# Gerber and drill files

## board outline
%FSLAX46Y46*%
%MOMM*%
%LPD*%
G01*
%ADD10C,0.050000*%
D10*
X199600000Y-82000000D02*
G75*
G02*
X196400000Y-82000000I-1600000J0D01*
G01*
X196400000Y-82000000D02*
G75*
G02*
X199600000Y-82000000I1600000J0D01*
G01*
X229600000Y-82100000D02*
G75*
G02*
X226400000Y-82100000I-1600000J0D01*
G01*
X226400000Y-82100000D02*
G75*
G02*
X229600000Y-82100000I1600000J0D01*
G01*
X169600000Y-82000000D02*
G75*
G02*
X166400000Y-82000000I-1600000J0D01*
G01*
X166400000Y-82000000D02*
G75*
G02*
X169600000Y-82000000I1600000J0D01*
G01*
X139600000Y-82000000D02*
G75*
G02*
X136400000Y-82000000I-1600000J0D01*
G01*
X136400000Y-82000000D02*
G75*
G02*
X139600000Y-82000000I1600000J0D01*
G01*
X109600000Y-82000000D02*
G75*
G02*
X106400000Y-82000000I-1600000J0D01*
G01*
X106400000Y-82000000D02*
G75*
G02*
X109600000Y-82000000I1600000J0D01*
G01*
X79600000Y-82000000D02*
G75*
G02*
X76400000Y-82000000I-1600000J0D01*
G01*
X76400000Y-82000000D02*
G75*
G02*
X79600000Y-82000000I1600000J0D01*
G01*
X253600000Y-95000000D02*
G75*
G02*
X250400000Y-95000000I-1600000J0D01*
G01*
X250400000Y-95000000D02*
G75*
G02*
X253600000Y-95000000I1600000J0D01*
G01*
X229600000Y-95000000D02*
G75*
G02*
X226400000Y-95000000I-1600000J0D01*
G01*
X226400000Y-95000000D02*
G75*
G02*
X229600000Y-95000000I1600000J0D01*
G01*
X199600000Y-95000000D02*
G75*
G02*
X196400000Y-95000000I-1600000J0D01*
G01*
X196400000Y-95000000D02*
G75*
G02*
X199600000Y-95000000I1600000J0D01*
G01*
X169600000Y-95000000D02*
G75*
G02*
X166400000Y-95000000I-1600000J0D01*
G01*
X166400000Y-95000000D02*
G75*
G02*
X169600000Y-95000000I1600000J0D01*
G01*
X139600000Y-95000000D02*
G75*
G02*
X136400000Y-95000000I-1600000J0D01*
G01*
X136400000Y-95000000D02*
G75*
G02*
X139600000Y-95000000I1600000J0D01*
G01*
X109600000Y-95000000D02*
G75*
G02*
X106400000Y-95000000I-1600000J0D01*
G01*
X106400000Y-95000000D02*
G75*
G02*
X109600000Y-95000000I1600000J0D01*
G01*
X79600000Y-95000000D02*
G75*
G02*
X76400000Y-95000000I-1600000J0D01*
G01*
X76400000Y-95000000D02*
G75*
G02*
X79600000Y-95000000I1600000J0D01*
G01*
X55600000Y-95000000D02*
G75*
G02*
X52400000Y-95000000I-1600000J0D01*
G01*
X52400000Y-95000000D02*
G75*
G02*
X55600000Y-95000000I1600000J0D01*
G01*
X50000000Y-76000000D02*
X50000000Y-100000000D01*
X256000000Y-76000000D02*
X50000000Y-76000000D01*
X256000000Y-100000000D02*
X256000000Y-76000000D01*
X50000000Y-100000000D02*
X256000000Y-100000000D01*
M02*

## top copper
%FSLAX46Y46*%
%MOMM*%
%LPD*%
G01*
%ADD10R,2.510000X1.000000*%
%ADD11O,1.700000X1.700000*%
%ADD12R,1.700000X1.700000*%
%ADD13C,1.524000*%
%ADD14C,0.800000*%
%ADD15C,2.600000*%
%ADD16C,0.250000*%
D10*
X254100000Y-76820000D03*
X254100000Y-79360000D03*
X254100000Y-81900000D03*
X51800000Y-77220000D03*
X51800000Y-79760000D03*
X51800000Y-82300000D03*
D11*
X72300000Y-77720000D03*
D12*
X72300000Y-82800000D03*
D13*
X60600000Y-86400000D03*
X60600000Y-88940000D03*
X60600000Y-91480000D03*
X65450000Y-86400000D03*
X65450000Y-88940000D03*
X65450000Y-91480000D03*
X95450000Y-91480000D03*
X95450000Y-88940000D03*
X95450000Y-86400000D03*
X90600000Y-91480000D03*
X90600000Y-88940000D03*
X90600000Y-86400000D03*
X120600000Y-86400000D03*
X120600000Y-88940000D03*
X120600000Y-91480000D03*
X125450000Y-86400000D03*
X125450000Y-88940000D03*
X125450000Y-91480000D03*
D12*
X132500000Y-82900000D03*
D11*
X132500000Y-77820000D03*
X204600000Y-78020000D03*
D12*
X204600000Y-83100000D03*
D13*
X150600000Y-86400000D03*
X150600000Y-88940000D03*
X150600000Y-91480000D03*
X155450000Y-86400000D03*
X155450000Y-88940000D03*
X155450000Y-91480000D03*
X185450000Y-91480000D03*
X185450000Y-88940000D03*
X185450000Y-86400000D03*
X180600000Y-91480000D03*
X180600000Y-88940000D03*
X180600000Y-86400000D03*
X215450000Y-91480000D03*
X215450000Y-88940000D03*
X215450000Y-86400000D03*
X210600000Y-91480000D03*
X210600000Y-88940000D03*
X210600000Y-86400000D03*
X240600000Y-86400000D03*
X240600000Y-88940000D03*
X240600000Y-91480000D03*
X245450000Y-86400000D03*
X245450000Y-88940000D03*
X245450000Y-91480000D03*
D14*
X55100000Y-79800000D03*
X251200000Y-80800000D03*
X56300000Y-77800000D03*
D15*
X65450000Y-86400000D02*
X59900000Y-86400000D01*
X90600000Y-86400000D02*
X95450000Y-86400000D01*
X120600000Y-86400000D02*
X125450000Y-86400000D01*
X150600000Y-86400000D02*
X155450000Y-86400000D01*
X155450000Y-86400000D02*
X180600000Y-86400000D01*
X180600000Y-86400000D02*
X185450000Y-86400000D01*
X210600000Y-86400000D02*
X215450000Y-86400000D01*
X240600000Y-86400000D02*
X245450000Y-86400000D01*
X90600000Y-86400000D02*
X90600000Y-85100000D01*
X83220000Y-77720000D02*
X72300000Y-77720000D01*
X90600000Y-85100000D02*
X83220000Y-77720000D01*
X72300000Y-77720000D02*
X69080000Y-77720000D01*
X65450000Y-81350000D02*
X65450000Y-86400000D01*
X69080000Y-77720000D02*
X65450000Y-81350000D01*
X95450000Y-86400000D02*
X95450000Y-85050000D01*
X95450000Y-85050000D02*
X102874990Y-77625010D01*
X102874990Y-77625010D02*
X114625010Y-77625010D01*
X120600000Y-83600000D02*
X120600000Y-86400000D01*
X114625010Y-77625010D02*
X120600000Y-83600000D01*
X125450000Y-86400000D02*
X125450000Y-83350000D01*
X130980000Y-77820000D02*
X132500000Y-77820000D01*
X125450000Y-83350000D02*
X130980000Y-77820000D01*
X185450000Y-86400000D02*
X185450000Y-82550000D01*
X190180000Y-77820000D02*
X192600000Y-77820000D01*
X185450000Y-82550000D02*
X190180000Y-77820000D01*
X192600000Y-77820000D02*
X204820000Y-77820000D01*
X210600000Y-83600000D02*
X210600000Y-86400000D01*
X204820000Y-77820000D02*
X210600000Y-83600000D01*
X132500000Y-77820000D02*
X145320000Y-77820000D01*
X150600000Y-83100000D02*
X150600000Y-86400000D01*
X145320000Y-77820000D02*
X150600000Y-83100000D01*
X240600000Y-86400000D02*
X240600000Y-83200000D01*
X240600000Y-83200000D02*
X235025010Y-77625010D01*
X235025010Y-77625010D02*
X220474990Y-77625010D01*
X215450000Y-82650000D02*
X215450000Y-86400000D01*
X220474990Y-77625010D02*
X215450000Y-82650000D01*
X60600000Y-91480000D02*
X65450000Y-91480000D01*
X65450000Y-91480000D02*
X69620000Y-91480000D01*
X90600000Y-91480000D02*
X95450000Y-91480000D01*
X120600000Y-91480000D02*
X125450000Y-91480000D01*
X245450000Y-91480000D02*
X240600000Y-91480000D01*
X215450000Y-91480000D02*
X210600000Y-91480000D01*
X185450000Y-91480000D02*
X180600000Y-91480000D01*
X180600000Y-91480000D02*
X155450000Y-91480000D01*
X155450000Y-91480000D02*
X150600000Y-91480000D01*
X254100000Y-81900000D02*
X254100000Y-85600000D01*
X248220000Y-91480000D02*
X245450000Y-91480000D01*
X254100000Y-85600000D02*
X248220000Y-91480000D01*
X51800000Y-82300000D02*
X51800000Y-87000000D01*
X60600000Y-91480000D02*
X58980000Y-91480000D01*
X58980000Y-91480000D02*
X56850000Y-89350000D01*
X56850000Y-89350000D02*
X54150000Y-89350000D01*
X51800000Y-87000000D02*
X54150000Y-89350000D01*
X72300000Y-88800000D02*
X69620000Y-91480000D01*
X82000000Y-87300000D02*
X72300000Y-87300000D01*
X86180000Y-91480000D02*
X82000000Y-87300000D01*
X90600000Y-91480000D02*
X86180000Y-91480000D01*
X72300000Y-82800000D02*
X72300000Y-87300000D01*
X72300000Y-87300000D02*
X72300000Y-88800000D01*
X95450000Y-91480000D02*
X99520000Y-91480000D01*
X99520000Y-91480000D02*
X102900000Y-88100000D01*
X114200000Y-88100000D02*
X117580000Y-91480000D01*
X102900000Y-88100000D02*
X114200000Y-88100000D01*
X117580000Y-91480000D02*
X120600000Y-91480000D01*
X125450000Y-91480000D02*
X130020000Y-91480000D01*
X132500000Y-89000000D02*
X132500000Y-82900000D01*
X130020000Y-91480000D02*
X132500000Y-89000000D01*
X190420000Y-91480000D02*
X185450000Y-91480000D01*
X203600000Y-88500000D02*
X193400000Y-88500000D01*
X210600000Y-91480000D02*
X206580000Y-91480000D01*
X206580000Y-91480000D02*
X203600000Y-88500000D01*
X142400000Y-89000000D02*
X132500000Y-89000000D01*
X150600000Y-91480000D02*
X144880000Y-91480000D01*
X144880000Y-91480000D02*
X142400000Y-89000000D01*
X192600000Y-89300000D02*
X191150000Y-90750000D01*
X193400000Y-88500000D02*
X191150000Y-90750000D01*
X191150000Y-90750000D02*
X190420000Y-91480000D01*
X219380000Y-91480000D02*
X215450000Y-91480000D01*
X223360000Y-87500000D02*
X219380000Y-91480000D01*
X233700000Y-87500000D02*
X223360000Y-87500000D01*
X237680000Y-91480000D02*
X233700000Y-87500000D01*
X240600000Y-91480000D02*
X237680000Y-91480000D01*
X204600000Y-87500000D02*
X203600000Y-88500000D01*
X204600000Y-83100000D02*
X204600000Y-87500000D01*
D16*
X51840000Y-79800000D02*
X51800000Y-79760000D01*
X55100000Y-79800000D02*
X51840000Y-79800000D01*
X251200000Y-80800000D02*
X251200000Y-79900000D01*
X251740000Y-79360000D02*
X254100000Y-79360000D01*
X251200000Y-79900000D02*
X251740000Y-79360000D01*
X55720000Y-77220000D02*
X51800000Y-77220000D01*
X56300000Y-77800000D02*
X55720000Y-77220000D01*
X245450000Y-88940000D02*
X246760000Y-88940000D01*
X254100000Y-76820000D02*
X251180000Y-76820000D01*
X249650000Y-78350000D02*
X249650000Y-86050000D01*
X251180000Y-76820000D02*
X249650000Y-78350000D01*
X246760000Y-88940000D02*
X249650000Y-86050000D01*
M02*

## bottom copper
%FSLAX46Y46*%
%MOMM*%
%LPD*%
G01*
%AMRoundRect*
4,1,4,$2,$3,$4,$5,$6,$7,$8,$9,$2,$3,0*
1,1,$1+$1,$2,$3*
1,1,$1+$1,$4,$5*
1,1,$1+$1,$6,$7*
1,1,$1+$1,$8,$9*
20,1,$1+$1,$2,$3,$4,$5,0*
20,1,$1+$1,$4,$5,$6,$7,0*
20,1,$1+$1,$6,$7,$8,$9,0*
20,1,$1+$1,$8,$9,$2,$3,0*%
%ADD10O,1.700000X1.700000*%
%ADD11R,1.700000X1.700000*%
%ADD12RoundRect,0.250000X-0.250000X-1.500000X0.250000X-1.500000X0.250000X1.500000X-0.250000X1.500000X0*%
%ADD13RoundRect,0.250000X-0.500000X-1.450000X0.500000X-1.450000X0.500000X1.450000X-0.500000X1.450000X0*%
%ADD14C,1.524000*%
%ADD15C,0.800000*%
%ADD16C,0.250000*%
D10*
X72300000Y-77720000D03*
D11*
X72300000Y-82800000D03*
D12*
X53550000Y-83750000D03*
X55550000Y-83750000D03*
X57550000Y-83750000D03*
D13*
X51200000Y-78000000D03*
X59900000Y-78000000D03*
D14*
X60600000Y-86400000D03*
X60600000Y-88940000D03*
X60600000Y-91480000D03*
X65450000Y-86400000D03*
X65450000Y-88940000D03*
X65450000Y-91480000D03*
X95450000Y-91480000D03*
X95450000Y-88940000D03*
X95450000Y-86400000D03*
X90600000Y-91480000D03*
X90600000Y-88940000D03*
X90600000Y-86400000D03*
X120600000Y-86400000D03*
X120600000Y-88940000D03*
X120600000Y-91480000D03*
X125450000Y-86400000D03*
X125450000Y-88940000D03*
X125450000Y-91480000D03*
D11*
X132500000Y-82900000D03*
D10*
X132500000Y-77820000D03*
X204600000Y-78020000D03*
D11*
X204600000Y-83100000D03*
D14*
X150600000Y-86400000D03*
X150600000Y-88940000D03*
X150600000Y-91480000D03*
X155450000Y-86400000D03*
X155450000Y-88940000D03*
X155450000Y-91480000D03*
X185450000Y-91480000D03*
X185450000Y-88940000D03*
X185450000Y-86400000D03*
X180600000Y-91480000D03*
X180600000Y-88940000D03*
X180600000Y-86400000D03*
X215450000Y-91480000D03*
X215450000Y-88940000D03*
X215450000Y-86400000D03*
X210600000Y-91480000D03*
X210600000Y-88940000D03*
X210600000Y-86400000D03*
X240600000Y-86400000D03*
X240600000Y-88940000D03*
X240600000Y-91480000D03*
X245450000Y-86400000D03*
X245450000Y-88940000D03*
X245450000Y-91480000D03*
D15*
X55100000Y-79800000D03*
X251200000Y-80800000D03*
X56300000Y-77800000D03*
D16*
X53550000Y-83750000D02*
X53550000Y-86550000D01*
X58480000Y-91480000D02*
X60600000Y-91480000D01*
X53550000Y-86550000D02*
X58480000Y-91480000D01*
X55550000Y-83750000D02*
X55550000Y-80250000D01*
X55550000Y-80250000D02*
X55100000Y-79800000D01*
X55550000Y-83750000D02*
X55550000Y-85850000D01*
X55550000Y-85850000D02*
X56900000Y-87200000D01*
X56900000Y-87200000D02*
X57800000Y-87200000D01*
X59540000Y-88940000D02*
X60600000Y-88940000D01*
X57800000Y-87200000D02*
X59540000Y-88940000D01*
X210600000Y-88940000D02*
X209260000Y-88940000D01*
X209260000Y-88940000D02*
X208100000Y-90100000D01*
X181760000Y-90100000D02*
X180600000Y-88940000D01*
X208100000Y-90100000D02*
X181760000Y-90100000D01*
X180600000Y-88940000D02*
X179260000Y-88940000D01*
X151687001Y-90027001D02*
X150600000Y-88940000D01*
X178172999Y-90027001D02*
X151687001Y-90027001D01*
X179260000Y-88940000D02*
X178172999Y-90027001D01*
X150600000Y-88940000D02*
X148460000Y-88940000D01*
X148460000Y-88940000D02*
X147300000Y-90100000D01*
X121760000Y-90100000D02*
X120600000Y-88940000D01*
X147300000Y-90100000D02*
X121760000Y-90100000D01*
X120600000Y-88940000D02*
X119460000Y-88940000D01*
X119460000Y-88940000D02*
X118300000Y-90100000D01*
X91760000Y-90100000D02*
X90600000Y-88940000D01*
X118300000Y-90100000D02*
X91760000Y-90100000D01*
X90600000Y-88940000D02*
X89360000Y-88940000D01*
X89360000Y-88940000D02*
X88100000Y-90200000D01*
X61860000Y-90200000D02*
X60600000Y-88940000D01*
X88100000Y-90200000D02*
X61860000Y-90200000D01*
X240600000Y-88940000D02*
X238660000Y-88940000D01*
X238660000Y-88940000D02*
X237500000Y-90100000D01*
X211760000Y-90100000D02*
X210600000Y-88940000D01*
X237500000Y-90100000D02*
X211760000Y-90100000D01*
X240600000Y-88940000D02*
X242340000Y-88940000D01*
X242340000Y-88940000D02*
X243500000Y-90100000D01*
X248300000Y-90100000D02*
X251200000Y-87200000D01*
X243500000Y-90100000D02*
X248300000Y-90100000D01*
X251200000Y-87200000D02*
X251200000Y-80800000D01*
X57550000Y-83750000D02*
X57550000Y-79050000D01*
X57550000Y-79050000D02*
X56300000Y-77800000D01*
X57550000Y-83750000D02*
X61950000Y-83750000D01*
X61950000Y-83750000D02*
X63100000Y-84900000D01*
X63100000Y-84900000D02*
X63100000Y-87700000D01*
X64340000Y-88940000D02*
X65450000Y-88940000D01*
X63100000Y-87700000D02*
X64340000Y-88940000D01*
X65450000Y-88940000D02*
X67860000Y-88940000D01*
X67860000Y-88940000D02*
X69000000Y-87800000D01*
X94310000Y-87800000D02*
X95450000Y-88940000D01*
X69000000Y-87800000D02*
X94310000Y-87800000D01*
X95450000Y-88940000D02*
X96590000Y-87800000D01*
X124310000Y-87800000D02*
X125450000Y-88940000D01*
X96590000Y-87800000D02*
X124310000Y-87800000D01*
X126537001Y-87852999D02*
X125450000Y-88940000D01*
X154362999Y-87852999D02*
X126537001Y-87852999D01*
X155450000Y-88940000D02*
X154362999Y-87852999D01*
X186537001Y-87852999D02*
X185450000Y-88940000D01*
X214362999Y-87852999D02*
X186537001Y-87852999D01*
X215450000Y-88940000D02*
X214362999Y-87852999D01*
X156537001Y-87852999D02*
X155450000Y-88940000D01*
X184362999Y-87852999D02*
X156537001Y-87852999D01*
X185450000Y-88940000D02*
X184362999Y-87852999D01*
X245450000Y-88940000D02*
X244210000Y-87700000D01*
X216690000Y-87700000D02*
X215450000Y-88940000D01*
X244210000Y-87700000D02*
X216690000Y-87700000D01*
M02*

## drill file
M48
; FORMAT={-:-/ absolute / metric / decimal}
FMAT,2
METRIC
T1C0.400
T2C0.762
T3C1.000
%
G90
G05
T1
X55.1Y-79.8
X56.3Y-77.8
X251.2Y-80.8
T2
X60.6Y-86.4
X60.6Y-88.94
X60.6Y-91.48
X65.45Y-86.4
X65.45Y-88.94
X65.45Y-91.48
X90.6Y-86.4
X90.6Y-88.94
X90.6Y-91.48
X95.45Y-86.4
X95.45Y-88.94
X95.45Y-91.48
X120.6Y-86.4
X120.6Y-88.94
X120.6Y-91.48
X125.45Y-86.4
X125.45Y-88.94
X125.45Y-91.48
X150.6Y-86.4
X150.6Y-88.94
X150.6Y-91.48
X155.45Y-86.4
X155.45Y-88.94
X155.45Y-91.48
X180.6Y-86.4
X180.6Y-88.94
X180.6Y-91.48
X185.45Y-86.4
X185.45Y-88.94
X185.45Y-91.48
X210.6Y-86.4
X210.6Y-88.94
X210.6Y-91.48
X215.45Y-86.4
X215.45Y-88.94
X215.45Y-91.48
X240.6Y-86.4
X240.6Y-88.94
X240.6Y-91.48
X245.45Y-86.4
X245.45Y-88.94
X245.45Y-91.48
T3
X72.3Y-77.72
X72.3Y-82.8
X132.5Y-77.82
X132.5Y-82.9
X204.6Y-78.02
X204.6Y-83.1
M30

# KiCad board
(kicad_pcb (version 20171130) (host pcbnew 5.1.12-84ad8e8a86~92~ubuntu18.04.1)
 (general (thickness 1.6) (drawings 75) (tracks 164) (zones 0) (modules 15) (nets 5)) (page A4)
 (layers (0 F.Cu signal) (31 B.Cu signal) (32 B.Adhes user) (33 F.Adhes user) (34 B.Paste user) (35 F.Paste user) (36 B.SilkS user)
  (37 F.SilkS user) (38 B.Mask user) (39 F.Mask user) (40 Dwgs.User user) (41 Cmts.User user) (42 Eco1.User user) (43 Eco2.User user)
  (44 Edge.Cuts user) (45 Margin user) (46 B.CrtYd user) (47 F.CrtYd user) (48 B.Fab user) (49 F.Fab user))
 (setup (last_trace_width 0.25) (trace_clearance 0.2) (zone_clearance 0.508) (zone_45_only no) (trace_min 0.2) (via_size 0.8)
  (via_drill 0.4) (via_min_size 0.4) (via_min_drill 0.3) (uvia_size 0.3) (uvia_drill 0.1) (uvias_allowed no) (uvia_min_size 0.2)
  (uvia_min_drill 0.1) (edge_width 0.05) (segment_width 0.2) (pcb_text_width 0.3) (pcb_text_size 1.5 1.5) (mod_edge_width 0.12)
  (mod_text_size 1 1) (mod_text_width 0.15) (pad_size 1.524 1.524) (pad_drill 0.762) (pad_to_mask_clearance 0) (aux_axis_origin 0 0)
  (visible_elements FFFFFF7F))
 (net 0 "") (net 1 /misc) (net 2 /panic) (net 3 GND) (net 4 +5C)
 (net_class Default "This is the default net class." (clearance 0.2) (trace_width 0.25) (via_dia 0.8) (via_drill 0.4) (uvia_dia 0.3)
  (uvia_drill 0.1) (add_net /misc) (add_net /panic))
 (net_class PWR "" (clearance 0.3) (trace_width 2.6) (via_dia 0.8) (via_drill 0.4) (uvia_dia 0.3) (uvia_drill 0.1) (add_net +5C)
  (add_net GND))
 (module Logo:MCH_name (layer F.Cu) (at 181.4 79.5)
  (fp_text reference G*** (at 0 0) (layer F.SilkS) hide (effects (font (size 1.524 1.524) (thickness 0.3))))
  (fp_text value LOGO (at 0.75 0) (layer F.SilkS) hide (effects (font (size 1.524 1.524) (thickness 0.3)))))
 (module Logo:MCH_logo (layer F.Cu) (at 162.3 79.5)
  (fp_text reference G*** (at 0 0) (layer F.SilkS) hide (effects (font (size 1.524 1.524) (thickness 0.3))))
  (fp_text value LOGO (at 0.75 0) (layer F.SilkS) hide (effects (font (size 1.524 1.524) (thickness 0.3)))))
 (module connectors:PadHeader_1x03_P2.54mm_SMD (layer F.Cu) (at 254.1 81.9 180)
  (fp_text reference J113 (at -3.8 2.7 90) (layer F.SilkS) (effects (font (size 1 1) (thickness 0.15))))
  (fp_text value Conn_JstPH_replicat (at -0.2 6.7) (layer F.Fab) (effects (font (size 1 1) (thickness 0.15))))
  (pad 3 smd rect (at 0 5.08 180) (size 2.51 1) (layers F.Cu F.Paste F.Mask) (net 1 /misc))
  (pad 2 smd rect (at 0 2.54 180) (size 2.51 1) (layers F.Cu F.Paste F.Mask) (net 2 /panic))
  (pad 1 smd rect (at 0 0 180) (size 2.51 1) (layers F.Cu F.Paste F.Mask) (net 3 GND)))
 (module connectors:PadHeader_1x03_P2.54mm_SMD (layer F.Cu) (at 51.8 82.3 180)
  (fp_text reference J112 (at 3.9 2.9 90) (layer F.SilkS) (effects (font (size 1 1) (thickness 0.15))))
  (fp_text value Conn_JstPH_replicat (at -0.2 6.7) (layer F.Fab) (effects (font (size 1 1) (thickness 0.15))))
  (pad 3 smd rect (at 0 5.08 180) (size 2.51 1) (layers F.Cu F.Paste F.Mask) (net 1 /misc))
  (pad 2 smd rect (at 0 2.54 180) (size 2.51 1) (layers F.Cu F.Paste F.Mask) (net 2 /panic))
  (pad 1 smd rect (at 0 0 180) (size 2.51 1) (layers F.Cu F.Paste F.Mask) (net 3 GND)))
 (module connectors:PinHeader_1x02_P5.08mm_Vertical (layer F.Cu) (at 72.3 82.8 180)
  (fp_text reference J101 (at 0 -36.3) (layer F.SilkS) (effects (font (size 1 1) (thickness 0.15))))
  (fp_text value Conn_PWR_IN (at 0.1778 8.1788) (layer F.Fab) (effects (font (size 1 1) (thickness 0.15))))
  (pad 2 thru_hole oval (at 0 5.08 180) (size 1.7 1.7) (drill 1) (layers *.Cu *.Mask) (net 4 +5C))
  (pad 1 thru_hole rect (at 0 0 180) (size 1.7 1.7) (drill 1) (layers *.Cu *.Mask) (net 3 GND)))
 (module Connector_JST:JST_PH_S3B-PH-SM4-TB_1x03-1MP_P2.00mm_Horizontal (layer B.Cu) (at 55.55 80.9)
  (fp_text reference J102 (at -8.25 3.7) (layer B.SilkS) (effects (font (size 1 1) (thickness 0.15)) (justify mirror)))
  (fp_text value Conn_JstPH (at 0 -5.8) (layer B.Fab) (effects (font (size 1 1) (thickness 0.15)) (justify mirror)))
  (pad 1 smd roundrect (at -2 2.85) (size 1 3.5) (layers B.Cu B.Paste B.Mask) (roundrect_rratio 0.25) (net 3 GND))
  (pad 2 smd roundrect (at 0 2.85) (size 1 3.5) (layers B.Cu B.Paste B.Mask) (roundrect_rratio 0.25) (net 2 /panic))
  (pad 3 smd roundrect (at 2 2.85) (size 1 3.5) (layers B.Cu B.Paste B.Mask) (roundrect_rratio 0.25) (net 1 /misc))
  (pad MP smd roundrect (at -4.35 -2.9) (size 1.5 3.4) (layers B.Cu B.Paste B.Mask) (roundrect_rratio 0.1666666666666667))
  (pad MP smd roundrect (at 4.35 -2.9) (size 1.5 3.4) (layers B.Cu B.Paste B.Mask) (roundrect_rratio 0.1666666666666667)))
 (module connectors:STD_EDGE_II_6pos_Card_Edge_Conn (layer F.Cu) (at 60.6 86.4)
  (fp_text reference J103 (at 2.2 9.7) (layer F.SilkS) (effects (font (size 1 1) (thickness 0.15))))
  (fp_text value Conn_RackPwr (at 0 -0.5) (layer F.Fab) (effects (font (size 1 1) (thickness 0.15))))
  (pad 1 thru_hole circle (at 0 0) (size 1.524 1.524) (drill 0.762) (layers *.Cu *.Mask) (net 4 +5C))
  (pad 2 thru_hole circle (at 0 2.54) (size 1.524 1.524) (drill 0.762) (layers *.Cu *.Mask) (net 2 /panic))
  (pad 3 thru_hole circle (at 0 5.08) (size 1.524 1.524) (drill 0.762) (layers *.Cu *.Mask) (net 3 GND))
  (pad 6 thru_hole circle (at 4.85 0) (size 1.524 1.524) (drill 0.762) (layers *.Cu *.Mask) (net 4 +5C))
  (pad 5 thru_hole circle (at 4.85 2.54) (size 1.524 1.524) (drill 0.762) (layers *.Cu *.Mask) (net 1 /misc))
  (pad 4 thru_hole circle (at 4.85 5.08) (size 1.524 1.524) (drill 0.762) (layers *.Cu *.Mask) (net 3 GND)))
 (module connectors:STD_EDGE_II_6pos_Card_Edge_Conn (layer F.Cu) (at 90.6 86.4)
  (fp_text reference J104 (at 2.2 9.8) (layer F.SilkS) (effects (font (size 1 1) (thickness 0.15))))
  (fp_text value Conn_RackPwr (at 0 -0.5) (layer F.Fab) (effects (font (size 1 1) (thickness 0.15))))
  (pad 4 thru_hole circle (at 4.85 5.08) (size 1.524 1.524) (drill 0.762) (layers *.Cu *.Mask) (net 3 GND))
  (pad 5 thru_hole circle (at 4.85 2.54) (size 1.524 1.524) (drill 0.762) (layers *.Cu *.Mask) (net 1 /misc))
  (pad 6 thru_hole circle (at 4.85 0) (size 1.524 1.524) (drill 0.762) (layers *.Cu *.Mask) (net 4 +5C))
  (pad 3 thru_hole circle (at 0 5.08) (size 1.524 1.524) (drill 0.762) (layers *.Cu *.Mask) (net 3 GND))
  (pad 2 thru_hole circle (at 0 2.54) (size 1.524 1.524) (drill 0.762) (layers *.Cu *.Mask) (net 2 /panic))
  (pad 1 thru_hole circle (at 0 0) (size 1.524 1.524) (drill 0.762) (layers *.Cu *.Mask) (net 4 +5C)))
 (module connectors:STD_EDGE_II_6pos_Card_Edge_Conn (layer F.Cu) (at 120.6 86.4)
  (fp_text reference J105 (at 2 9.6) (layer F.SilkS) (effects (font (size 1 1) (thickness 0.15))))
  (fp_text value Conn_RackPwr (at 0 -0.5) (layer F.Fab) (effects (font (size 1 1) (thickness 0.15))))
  (pad 1 thru_hole circle (at 0 0) (size 1.524 1.524) (drill 0.762) (layers *.Cu *.Mask) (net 4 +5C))
  (pad 2 thru_hole circle (at 0 2.54) (size 1.524 1.524) (drill 0.762) (layers *.Cu *.Mask) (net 2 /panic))
  (pad 3 thru_hole circle (at 0 5.08) (size 1.524 1.524) (drill 0.762) (layers *.Cu *.Mask) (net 3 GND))
  (pad 6 thru_hole circle (at 4.85 0) (size 1.524 1.524) (drill 0.762) (layers *.Cu *.Mask) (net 4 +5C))
  (pad 5 thru_hole circle (at 4.85 2.54) (size 1.524 1.524) (drill 0.762) (layers *.Cu *.Mask) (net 1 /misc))
  (pad 4 thru_hole circle (at 4.85 5.08) (size 1.524 1.524) (drill 0.762) (layers *.Cu *.Mask) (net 3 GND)))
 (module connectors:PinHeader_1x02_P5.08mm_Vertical (layer F.Cu) (at 132.5 82.9 180)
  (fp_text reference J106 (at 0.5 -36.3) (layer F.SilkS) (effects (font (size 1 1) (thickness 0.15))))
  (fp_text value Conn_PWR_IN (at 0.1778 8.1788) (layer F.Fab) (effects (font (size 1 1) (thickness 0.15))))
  (pad 1 thru_hole rect (at 0 0 180) (size 1.7 1.7) (drill 1) (layers *.Cu *.Mask) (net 3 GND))
  (pad 2 thru_hole oval (at 0 5.08 180) (size 1.7 1.7) (drill 1) (layers *.Cu *.Mask) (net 4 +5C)))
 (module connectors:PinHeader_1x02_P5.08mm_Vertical (layer F.Cu) (at 204.6 83.1 180)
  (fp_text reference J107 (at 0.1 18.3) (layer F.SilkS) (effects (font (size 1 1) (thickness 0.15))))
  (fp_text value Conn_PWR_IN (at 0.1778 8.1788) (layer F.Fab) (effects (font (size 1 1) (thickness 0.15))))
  (pad 2 thru_hole oval (at 0 5.08 180) (size 1.7 1.7) (drill 1) (layers *.Cu *.Mask) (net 4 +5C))
  (pad 1 thru_hole rect (at 0 0 180) (size 1.7 1.7) (drill 1) (layers *.Cu *.Mask) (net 3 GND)))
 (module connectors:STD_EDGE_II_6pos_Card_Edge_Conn (layer F.Cu) (at 150.6 86.4)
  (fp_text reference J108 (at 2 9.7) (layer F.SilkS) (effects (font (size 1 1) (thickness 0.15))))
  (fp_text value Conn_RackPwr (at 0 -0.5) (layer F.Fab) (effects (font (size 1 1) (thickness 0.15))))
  (pad 1 thru_hole circle (at 0 0) (size 1.524 1.524) (drill 0.762) (layers *.Cu *.Mask) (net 4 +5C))
  (pad 2 thru_hole circle (at 0 2.54) (size 1.524 1.524) (drill 0.762) (layers *.Cu *.Mask) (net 2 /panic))
  (pad 3 thru_hole circle (at 0 5.08) (size 1.524 1.524) (drill 0.762) (layers *.Cu *.Mask) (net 3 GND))
  (pad 6 thru_hole circle (at 4.85 0) (size 1.524 1.524) (drill 0.762) (layers *.Cu *.Mask) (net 4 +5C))
  (pad 5 thru_hole circle (at 4.85 2.54) (size 1.524 1.524) (drill 0.762) (layers *.Cu *.Mask) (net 1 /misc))
  (pad 4 thru_hole circle (at 4.85 5.08) (size 1.524 1.524) (drill 0.762) (layers *.Cu *.Mask) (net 3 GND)))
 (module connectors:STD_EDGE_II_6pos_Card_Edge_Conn (layer F.Cu) (at 180.6 86.4)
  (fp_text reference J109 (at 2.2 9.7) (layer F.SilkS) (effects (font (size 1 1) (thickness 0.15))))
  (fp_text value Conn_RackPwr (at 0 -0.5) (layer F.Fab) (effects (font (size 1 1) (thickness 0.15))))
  (pad 4 thru_hole circle (at 4.85 5.08) (size 1.524 1.524) (drill 0.762) (layers *.Cu *.Mask) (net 3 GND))
  (pad 5 thru_hole circle (at 4.85 2.54) (size 1.524 1.524) (drill 0.762) (layers *.Cu *.Mask) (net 1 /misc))
  (pad 6 thru_hole circle (at 4.85 0) (size 1.524 1.524) (drill 0.762) (layers *.Cu *.Mask) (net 4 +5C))
  (pad 3 thru_hole circle (at 0 5.08) (size 1.524 1.524) (drill 0.762) (layers *.Cu *.Mask) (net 3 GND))
  (pad 2 thru_hole circle (at 0 2.54) (size 1.524 1.524) (drill 0.762) (layers *.Cu *.Mask) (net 2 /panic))
  (pad 1 thru_hole circle (at 0 0) (size 1.524 1.524) (drill 0.762) (layers *.Cu *.Mask) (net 4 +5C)))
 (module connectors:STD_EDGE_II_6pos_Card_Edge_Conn (layer F.Cu) (at 210.6 86.4)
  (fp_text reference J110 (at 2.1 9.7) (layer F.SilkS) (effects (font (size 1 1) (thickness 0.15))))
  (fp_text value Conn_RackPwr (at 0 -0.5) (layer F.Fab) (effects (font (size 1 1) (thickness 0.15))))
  (pad 4 thru_hole circle (at 4.85 5.08) (size 1.524 1.524) (drill 0.762) (layers *.Cu *.Mask) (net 3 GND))
  (pad 5 thru_hole circle (at 4.85 2.54) (size 1.524 1.524) (drill 0.762) (layers *.Cu *.Mask) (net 1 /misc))
  (pad 6 thru_hole circle (at 4.85 0) (size 1.524 1.524) (drill 0.762) (layers *.Cu *.Mask) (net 4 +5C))
  (pad 3 thru_hole circle (at 0 5.08) (size 1.524 1.524) (drill 0.762) (layers *.Cu *.Mask) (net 3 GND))
  (pad 2 thru_hole circle (at 0 2.54) (size 1.524 1.524) (drill 0.762) (layers *.Cu *.Mask) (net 2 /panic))
  (pad 1 thru_hole circle (at 0 0) (size 1.524 1.524) (drill 0.762) (layers *.Cu *.Mask) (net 4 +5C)))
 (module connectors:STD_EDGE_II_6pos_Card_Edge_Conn (layer F.Cu) (at 240.6 86.4)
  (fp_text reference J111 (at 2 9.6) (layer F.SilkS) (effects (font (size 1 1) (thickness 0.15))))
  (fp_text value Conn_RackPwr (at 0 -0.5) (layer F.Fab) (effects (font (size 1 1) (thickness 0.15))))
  (pad 1 thru_hole circle (at 0 0) (size 1.524 1.524) (drill 0.762) (layers *.Cu *.Mask) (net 4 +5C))
  (pad 2 thru_hole circle (at 0 2.54) (size 1.524 1.524) (drill 0.762) (layers *.Cu *.Mask) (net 2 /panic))
  (pad 3 thru_hole circle (at 0 5.08) (size 1.524 1.524) (drill 0.762) (layers *.Cu *.Mask) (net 3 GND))
  (pad 6 thru_hole circle (at 4.85 0) (size 1.524 1.524) (drill 0.762) (layers *.Cu *.Mask) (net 4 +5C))
  (pad 5 thru_hole circle (at 4.85 2.54) (size 1.524 1.524) (drill 0.762) (layers *.Cu *.Mask) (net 1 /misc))
  (pad 4 thru_hole circle (at 4.85 5.08) (size 1.524 1.524) (drill 0.762) (layers *.Cu *.Mask) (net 3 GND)))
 (gr_circle (center 198 82) (end 199.6 82) (layer Edge.Cuts) (width 0.05))
 (gr_circle (center 228 82.1) (end 229.6 82.1) (layer Edge.Cuts) (width 0.05))
 (gr_circle (center 168 82) (end 169.6 82) (layer Edge.Cuts) (width 0.05))
 (gr_circle (center 138 82) (end 139.6 82) (layer Edge.Cuts) (width 0.05))
 (gr_circle (center 108 82) (end 109.6 82) (layer Edge.Cuts) (width 0.05))
 (gr_circle (center 78 82) (end 79.6 82) (layer Edge.Cuts) (width 0.05))
 (gr_circle (center 252 95) (end 253.6 95) (layer Edge.Cuts) (width 0.05))
 (gr_circle (center 228 95) (end 229.6 95) (layer Edge.Cuts) (width 0.05))
 (gr_circle (center 198 95) (end 199.6 95) (layer Edge.Cuts) (width 0.05))
 (gr_circle (center 168 95) (end 169.6 95) (layer Edge.Cuts) (width 0.05))
 (gr_circle (center 138 95) (end 139.6 95) (layer Edge.Cuts) (width 0.05))
 (gr_circle (center 108 95) (end 109.6 95) (layer Edge.Cuts) (width 0.05))
 (gr_circle (center 78 95) (end 79.6 95) (layer Edge.Cuts) (width 0.05))
 (gr_circle (center 54 95) (end 55.6 95) (layer Edge.Cuts) (width 0.05))
 (gr_line (start 50 76) (end 50 100) (layer Edge.Cuts) (width 0.05))
 (gr_line (start 256 76) (end 50 76) (layer Edge.Cuts) (width 0.05))
 (gr_line (start 256 100) (end 256 76) (layer Edge.Cuts) (width 0.05))
 (gr_line (start 50 100) (end 256 100) (layer Edge.Cuts) (width 0.05))
 (segment (start 65.45 86.4) (end 59.9 86.4) (width 2.6) (layer F.Cu) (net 4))
 (segment (start 90.6 86.4) (end 95.45 86.4) (width 2.6) (layer F.Cu) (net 4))
 (segment (start 120.6 86.4) (end 125.45 86.4) (width 2.6) (layer F.Cu) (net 4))
 (segment (start 150.6 86.4) (end 155.45 86.4) (width 2.6) (layer F.Cu) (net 4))
 (segment (start 155.45 86.4) (end 180.6 86.4) (width 2.6) (layer F.Cu) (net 4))
 (segment (start 180.6 86.4) (end 185.45 86.4) (width 2.6) (layer F.Cu) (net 4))
 (segment (start 210.6 86.4) (end 215.45 86.4) (width 2.6) (layer F.Cu) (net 4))
 (segment (start 240.6 86.4) (end 245.45 86.4) (width 2.6) (layer F.Cu) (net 4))
 (segment (start 90.6 86.4) (end 90.6 85.1) (width 2.6) (layer F.Cu) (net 4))
 (segment (start 83.22 77.72) (end 72.3 77.72) (width 2.6) (layer F.Cu) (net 4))
 (segment (start 90.6 85.1) (end 83.22 77.72) (width 2.6) (layer F.Cu) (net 4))
 (segment (start 72.3 77.72) (end 69.08 77.72) (width 2.6) (layer F.Cu) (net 4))
 (segment (start 65.45 81.35) (end 65.45 86.4) (width 2.6) (layer F.Cu) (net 4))
 (segment (start 69.08 77.72) (end 65.45 81.35) (width 2.6) (layer F.Cu) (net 4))
 (segment (start 95.45 86.4) (end 95.45 85.05) (width 2.6) (layer F.Cu) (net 4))
 (segment (start 95.45 85.05) (end 102.87499 77.62501) (width 2.6) (layer F.Cu) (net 4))
 (segment (start 102.87499 77.62501) (end 114.62501 77.62501) (width 2.6) (layer F.Cu) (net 4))
 (segment (start 120.6 83.6) (end 120.6 86.4) (width 2.6) (layer F.Cu) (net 4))
 (segment (start 114.62501 77.62501) (end 120.6 83.6) (width 2.6) (layer F.Cu) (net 4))
 (segment (start 125.45 86.4) (end 125.45 83.35) (width 2.6) (layer F.Cu) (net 4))
 (segment (start 130.98 77.82) (end 132.5 77.82) (width 2.6) (layer F.Cu) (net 4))
 (segment (start 125.45 83.35) (end 130.98 77.82) (width 2.6) (layer F.Cu) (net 4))
 (segment (start 185.45 86.4) (end 185.45 82.55) (width 2.6) (layer F.Cu) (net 4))
 (segment (start 190.18 77.82) (end 192.6 77.82) (width 2.6) (layer F.Cu) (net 4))
 (segment (start 185.45 82.55) (end 190.18 77.82) (width 2.6) (layer F.Cu) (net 4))
 (segment (start 192.6 77.82) (end 204.82 77.82) (width 2.6) (layer F.Cu) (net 4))
 (segment (start 210.6 83.6) (end 210.6 86.4) (width 2.6) (layer F.Cu) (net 4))
 (segment (start 204.82 77.82) (end 210.6 83.6) (width 2.6) (layer F.Cu) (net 4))
 (segment (start 132.5 77.82) (end 145.32 77.82) (width 2.6) (layer F.Cu) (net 4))
 (segment (start 150.6 83.1) (end 150.6 86.4) (width 2.6) (layer F.Cu) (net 4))
 (segment (start 145.32 77.82) (end 150.6 83.1) (width 2.6) (layer F.Cu) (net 4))
 (segment (start 240.6 86.4) (end 240.6 83.2) (width 2.6) (layer F.Cu) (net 4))
 (segment (start 240.6 83.2) (end 235.02501 77.62501) (width 2.6) (layer F.Cu) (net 4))
 (segment (start 235.02501 77.62501) (end 220.47499 77.62501) (width 2.6) (layer F.Cu) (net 4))
 (segment (start 215.45 82.65) (end 215.45 86.4) (width 2.6) (layer F.Cu) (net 4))
 (segment (start 220.47499 77.62501) (end 215.45 82.65) (width 2.6) (layer F.Cu) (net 4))
 (segment (start 60.6 91.48) (end 65.45 91.48) (width 2.6) (layer F.Cu) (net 3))
 (segment (start 65.45 91.48) (end 69.62 91.48) (width 2.6) (layer F.Cu) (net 3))
 (segment (start 90.6 91.48) (end 95.45 91.48) (width 2.6) (layer F.Cu) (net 3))
 (segment (start 120.6 91.48) (end 125.45 91.48) (width 2.6) (layer F.Cu) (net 3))
 (segment (start 245.45 91.48) (end 240.6 91.48) (width 2.6) (layer F.Cu) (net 3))
 (segment (start 215.45 91.48) (end 210.6 91.48) (width 2.6) (layer F.Cu) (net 3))
 (segment (start 185.45 91.48) (end 180.6 91.48) (width 2.6) (layer F.Cu) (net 3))
 (segment (start 180.6 91.48) (end 155.45 91.48) (width 2.6) (layer F.Cu) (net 3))
 (segment (start 155.45 91.48) (end 150.6 91.48) (width 2.6) (layer F.Cu) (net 3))
 (segment (start 254.1 81.9) (end 254.1 85.6) (width 2.6) (layer F.Cu) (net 3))
 (segment (start 248.22 91.48) (end 245.45 91.48) (width 2.6) (layer F.Cu) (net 3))
 (segment (start 254.1 85.6) (end 248.22 91.48) (width 2.6) (layer F.Cu) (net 3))
 (segment (start 51.8 82.3) (end 51.8 87) (width 2.6) (layer F.Cu) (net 3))
 (segment (start 60.6 91.48) (end 58.98 91.48) (width 2.6) (layer F.Cu) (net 3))
 (segment (start 58.98 91.48) (end 56.85 89.35) (width 2.6) (layer F.Cu) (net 3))
 (segment (start 56.85 89.35) (end 54.15 89.35) (width 2.6) (layer F.Cu) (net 3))
 (segment (start 51.8 87) (end 54.15 89.35) (width 2.6) (layer F.Cu) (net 3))
 (segment (start 53.55 83.75) (end 53.55 86.55) (width 0.25) (layer B.Cu) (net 3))
 (segment (start 58.48 91.48) (end 60.6 91.48) (width 0.25) (layer B.Cu) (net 3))
 (segment (start 53.55 86.55) (end 58.48 91.48) (width 0.25) (layer B.Cu) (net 3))
 (segment (start 72.3 88.8) (end 69.62 91.48) (width 2.6) (layer F.Cu) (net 3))
 (segment (start 82 87.3) (end 72.3 87.3) (width 2.6) (layer F.Cu) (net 3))
 (segment (start 86.18 91.48) (end 82 87.3) (width 2.6) (layer F.Cu) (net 3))
 (segment (start 90.6 91.48) (end 86.18 91.48) (width 2.6) (layer F.Cu) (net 3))
 (segment (start 72.3 82.8) (end 72.3 87.3) (width 2.6) (layer F.Cu) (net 3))
 (segment (start 72.3 87.3) (end 72.3 88.8) (width 2.6) (layer F.Cu) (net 3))
 (segment (start 95.45 91.48) (end 99.52 91.48) (width 2.6) (layer F.Cu) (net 3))
 (segment (start 99.52 91.48) (end 102.9 88.1) (width 2.6) (layer F.Cu) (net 3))
 (segment (start 114.2 88.1) (end 117.58 91.48) (width 2.6) (layer F.Cu) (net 3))
 (segment (start 102.9 88.1) (end 114.2 88.1) (width 2.6) (layer F.Cu) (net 3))
 (segment (start 117.58 91.48) (end 120.6 91.48) (width 2.6) (layer F.Cu) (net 3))
 (segment (start 125.45 91.48) (end 130.02 91.48) (width 2.6) (layer F.Cu) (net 3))
 (segment (start 132.5 89) (end 132.5 82.9) (width 2.6) (layer F.Cu) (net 3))
 (segment (start 130.02 91.48) (end 132.5 89) (width 2.6) (layer F.Cu) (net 3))
 (segment (start 190.42 91.48) (end 185.45 91.48) (width 2.6) (layer F.Cu) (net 3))
 (segment (start 203.6 88.5) (end 193.4 88.5) (width 2.6) (layer F.Cu) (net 3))
 (segment (start 210.6 91.48) (end 206.58 91.48) (width 2.6) (layer F.Cu) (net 3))
 (segment (start 206.58 91.48) (end 203.6 88.5) (width 2.6) (layer F.Cu) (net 3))
 (segment (start 142.4 89) (end 132.5 89) (width 2.6) (layer F.Cu) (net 3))
 (segment (start 150.6 91.48) (end 144.88 91.48) (width 2.6) (layer F.Cu) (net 3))
 (segment (start 144.88 91.48) (end 142.4 89) (width 2.6) (layer F.Cu) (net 3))
 (segment (start 192.6 89.3) (end 191.15 90.75) (width 2.6) (layer F.Cu) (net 3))
 (segment (start 193.4 88.5) (end 191.15 90.75) (width 2.6) (layer F.Cu) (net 3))
 (segment (start 191.15 90.75) (end 190.42 91.48) (width 2.6) (layer F.Cu) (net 3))
 (segment (start 219.38 91.48) (end 215.45 91.48) (width 2.6) (layer F.Cu) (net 3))
 (segment (start 223.36 87.5) (end 219.38 91.48) (width 2.6) (layer F.Cu) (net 3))
 (segment (start 233.7 87.5) (end 223.36 87.5) (width 2.6) (layer F.Cu) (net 3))
 (segment (start 237.68 91.48) (end 233.7 87.5) (width 2.6) (layer F.Cu) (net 3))
 (segment (start 240.6 91.48) (end 237.68 91.48) (width 2.6) (layer F.Cu) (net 3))
 (segment (start 204.6 87.5) (end 203.6 88.5) (width 2.6) (layer F.Cu) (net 3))
 (segment (start 204.6 83.1) (end 204.6 87.5) (width 2.6) (layer F.Cu) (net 3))
 (via (at 55.1 79.8) (size 0.8) (drill 0.4) (layers F.Cu B.Cu) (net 2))
 (segment (start 55.55 83.75) (end 55.55 80.25) (width 0.25) (layer B.Cu) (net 2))
 (segment (start 55.55 80.25) (end 55.1 79.8) (width 0.25) (layer B.Cu) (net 2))
 (segment (start 51.84 79.8) (end 51.8 79.76) (width 0.25) (layer F.Cu) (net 2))
 (segment (start 55.1 79.8) (end 51.84 79.8) (width 0.25) (layer F.Cu) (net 2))
 (segment (start 55.55 83.75) (end 55.55 85.85) (width 0.25) (layer B.Cu) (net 2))
 (segment (start 55.55 85.85) (end 56.9 87.2) (width 0.25) (layer B.Cu) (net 2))
 (segment (start 56.9 87.2) (end 57.8 87.2) (width 0.25) (layer B.Cu) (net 2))
 (segment (start 59.54 88.94) (end 60.6 88.94) (width 0.25) (layer B.Cu) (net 2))
 (segment (start 57.8 87.2) (end 59.54 88.94) (width 0.25) (layer B.Cu) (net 2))
 (via (at 251.2 80.8) (size 0.8) (drill 0.4) (layers F.Cu B.Cu) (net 2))
 (segment (start 251.2 80.8) (end 251.2 79.9) (width 0.25) (layer F.Cu) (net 2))
 (segment (start 251.74 79.36) (end 254.1 79.36) (width 0.25) (layer F.Cu) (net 2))
 (segment (start 251.2 79.9) (end 251.74 79.36) (width 0.25) (layer F.Cu) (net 2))
 (segment (start 210.6 88.94) (end 209.26 88.94) (width 0.25) (layer B.Cu) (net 2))
 (segment (start 209.26 88.94) (end 208.1 90.1) (width 0.25) (layer B.Cu) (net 2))
 (segment (start 181.76 90.1) (end 180.6 88.94) (width 0.25) (layer B.Cu) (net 2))
 (segment (start 208.1 90.1) (end 181.76 90.1) (width 0.25) (layer B.Cu) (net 2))
 (segment (start 180.6 88.94) (end 179.26 88.94) (width 0.25) (layer B.Cu) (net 2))
 (segment (start 151.687001 90.027001) (end 150.6 88.94) (width 0.25) (layer B.Cu) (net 2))
 (segment (start 178.172999 90.027001) (end 151.687001 90.027001) (width 0.25) (layer B.Cu) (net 2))
 (segment (start 179.26 88.94) (end 178.172999 90.027001) (width 0.25) (layer B.Cu) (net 2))
 (segment (start 150.6 88.94) (end 148.46 88.94) (width 0.25) (layer B.Cu) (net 2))
 (segment (start 148.46 88.94) (end 147.3 90.1) (width 0.25) (layer B.Cu) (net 2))
 (segment (start 121.76 90.1) (end 120.6 88.94) (width 0.25) (layer B.Cu) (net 2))
 (segment (start 147.3 90.1) (end 121.76 90.1) (width 0.25) (layer B.Cu) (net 2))
 (segment (start 120.6 88.94) (end 119.46 88.94) (width 0.25) (layer B.Cu) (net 2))
 (segment (start 119.46 88.94) (end 118.3 90.1) (width 0.25) (layer B.Cu) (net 2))
 (segment (start 91.76 90.1) (end 90.6 88.94) (width 0.25) (layer B.Cu) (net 2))
 (segment (start 118.3 90.1) (end 91.76 90.1) (width 0.25) (layer B.Cu) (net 2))
 (segment (start 90.6 88.94) (end 89.36 88.94) (width 0.25) (layer B.Cu) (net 2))
 (segment (start 89.36 88.94) (end 88.1 90.2) (width 0.25) (layer B.Cu) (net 2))
 (segment (start 61.86 90.2) (end 60.6 88.94) (width 0.25) (layer B.Cu) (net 2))
 (segment (start 88.1 90.2) (end 61.86 90.2) (width 0.25) (layer B.Cu) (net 2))
 (segment (start 240.6 88.94) (end 238.66 88.94) (width 0.25) (layer B.Cu) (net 2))
 (segment (start 238.66 88.94) (end 237.5 90.1) (width 0.25) (layer B.Cu) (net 2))
 (segment (start 211.76 90.1) (end 210.6 88.94) (width 0.25) (layer B.Cu) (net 2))
 (segment (start 237.5 90.1) (end 211.76 90.1) (width 0.25) (layer B.Cu) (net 2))
 (segment (start 240.6 88.94) (end 242.34 88.94) (width 0.25) (layer B.Cu) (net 2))
 (segment (start 242.34 88.94) (end 243.5 90.1) (width 0.25) (layer B.Cu) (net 2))
 (segment (start 248.3 90.1) (end 251.2 87.2) (width 0.25) (layer B.Cu) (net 2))
 (segment (start 243.5 90.1) (end 248.3 90.1) (width 0.25) (layer B.Cu) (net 2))
 (segment (start 251.2 87.2) (end 251.2 80.8) (width 0.25) (layer B.Cu) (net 2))
 (via (at 56.3 77.8) (size 0.8) (drill 0.4) (layers F.Cu B.Cu) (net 1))
 (segment (start 57.55 83.75) (end 57.55 79.05) (width 0.25) (layer B.Cu) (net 1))
 (segment (start 57.55 79.05) (end 56.3 77.8) (width 0.25) (layer B.Cu) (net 1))
 (segment (start 55.72 77.22) (end 51.8 77.22) (width 0.25) (layer F.Cu) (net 1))
 (segment (start 56.3 77.8) (end 55.72 77.22) (width 0.25) (layer F.Cu) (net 1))
 (segment (start 57.55 83.75) (end 61.95 83.75) (width 0.25) (layer B.Cu) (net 1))
 (segment (start 61.95 83.75) (end 63.1 84.9) (width 0.25) (layer B.Cu) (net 1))
 (segment (start 63.1 84.9) (end 63.1 87.7) (width 0.25) (layer B.Cu) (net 1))
 (segment (start 64.34 88.94) (end 65.45 88.94) (width 0.25) (layer B.Cu) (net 1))
 (segment (start 63.1 87.7) (end 64.34 88.94) (width 0.25) (layer B.Cu) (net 1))
 (segment (start 65.45 88.94) (end 67.86 88.94) (width 0.25) (layer B.Cu) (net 1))
 (segment (start 67.86 88.94) (end 69 87.8) (width 0.25) (layer B.Cu) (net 1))
 (segment (start 94.31 87.8) (end 95.45 88.94) (width 0.25) (layer B.Cu) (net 1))
 (segment (start 69 87.8) (end 94.31 87.8) (width 0.25) (layer B.Cu) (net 1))
 (segment (start 95.45 88.94) (end 96.59 87.8) (width 0.25) (layer B.Cu) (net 1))
 (segment (start 124.31 87.8) (end 125.45 88.94) (width 0.25) (layer B.Cu) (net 1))
 (segment (start 96.59 87.8) (end 124.31 87.8) (width 0.25) (layer B.Cu) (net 1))
 (segment (start 126.537001 87.852999) (end 125.45 88.94) (width 0.25) (layer B.Cu) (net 1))
 (segment (start 154.362999 87.852999) (end 126.537001 87.852999) (width 0.25) (layer B.Cu) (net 1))
 (segment (start 155.45 88.94) (end 154.362999 87.852999) (width 0.25) (layer B.Cu) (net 1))
 (segment (start 186.537001 87.852999) (end 185.45 88.94) (width 0.25) (layer B.Cu) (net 1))
 (segment (start 214.362999 87.852999) (end 186.537001 87.852999) (width 0.25) (layer B.Cu) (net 1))
 (segment (start 215.45 88.94) (end 214.362999 87.852999) (width 0.25) (layer B.Cu) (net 1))
 (segment (start 156.537001 87.852999) (end 155.45 88.94) (width 0.25) (layer B.Cu) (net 1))
 (segment (start 184.362999 87.852999) (end 156.537001 87.852999) (width 0.25) (layer B.Cu) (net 1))
 (segment (start 185.45 88.94) (end 184.362999 87.852999) (width 0.25) (layer B.Cu) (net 1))
 (segment (start 245.45 88.94) (end 244.21 87.7) (width 0.25) (layer B.Cu) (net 1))
 (segment (start 216.69 87.7) (end 215.45 88.94) (width 0.25) (layer B.Cu) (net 1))
 (segment (start 244.21 87.7) (end 216.69 87.7) (width 0.25) (layer B.Cu) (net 1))
 (segment (start 245.45 88.94) (end 246.76 88.94) (width 0.25) (layer F.Cu) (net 1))
 (segment (start 254.1 76.82) (end 251.18 76.82) (width 0.25) (layer F.Cu) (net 1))
 (segment (start 249.65 78.35) (end 249.65 86.05) (width 0.25) (layer F.Cu) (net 1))
 (segment (start 251.18 76.82) (end 249.65 78.35) (width 0.25) (layer F.Cu) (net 1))
 (segment (start 246.76 88.94) (end 249.65 86.05) (width 0.25) (layer F.Cu) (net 1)))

